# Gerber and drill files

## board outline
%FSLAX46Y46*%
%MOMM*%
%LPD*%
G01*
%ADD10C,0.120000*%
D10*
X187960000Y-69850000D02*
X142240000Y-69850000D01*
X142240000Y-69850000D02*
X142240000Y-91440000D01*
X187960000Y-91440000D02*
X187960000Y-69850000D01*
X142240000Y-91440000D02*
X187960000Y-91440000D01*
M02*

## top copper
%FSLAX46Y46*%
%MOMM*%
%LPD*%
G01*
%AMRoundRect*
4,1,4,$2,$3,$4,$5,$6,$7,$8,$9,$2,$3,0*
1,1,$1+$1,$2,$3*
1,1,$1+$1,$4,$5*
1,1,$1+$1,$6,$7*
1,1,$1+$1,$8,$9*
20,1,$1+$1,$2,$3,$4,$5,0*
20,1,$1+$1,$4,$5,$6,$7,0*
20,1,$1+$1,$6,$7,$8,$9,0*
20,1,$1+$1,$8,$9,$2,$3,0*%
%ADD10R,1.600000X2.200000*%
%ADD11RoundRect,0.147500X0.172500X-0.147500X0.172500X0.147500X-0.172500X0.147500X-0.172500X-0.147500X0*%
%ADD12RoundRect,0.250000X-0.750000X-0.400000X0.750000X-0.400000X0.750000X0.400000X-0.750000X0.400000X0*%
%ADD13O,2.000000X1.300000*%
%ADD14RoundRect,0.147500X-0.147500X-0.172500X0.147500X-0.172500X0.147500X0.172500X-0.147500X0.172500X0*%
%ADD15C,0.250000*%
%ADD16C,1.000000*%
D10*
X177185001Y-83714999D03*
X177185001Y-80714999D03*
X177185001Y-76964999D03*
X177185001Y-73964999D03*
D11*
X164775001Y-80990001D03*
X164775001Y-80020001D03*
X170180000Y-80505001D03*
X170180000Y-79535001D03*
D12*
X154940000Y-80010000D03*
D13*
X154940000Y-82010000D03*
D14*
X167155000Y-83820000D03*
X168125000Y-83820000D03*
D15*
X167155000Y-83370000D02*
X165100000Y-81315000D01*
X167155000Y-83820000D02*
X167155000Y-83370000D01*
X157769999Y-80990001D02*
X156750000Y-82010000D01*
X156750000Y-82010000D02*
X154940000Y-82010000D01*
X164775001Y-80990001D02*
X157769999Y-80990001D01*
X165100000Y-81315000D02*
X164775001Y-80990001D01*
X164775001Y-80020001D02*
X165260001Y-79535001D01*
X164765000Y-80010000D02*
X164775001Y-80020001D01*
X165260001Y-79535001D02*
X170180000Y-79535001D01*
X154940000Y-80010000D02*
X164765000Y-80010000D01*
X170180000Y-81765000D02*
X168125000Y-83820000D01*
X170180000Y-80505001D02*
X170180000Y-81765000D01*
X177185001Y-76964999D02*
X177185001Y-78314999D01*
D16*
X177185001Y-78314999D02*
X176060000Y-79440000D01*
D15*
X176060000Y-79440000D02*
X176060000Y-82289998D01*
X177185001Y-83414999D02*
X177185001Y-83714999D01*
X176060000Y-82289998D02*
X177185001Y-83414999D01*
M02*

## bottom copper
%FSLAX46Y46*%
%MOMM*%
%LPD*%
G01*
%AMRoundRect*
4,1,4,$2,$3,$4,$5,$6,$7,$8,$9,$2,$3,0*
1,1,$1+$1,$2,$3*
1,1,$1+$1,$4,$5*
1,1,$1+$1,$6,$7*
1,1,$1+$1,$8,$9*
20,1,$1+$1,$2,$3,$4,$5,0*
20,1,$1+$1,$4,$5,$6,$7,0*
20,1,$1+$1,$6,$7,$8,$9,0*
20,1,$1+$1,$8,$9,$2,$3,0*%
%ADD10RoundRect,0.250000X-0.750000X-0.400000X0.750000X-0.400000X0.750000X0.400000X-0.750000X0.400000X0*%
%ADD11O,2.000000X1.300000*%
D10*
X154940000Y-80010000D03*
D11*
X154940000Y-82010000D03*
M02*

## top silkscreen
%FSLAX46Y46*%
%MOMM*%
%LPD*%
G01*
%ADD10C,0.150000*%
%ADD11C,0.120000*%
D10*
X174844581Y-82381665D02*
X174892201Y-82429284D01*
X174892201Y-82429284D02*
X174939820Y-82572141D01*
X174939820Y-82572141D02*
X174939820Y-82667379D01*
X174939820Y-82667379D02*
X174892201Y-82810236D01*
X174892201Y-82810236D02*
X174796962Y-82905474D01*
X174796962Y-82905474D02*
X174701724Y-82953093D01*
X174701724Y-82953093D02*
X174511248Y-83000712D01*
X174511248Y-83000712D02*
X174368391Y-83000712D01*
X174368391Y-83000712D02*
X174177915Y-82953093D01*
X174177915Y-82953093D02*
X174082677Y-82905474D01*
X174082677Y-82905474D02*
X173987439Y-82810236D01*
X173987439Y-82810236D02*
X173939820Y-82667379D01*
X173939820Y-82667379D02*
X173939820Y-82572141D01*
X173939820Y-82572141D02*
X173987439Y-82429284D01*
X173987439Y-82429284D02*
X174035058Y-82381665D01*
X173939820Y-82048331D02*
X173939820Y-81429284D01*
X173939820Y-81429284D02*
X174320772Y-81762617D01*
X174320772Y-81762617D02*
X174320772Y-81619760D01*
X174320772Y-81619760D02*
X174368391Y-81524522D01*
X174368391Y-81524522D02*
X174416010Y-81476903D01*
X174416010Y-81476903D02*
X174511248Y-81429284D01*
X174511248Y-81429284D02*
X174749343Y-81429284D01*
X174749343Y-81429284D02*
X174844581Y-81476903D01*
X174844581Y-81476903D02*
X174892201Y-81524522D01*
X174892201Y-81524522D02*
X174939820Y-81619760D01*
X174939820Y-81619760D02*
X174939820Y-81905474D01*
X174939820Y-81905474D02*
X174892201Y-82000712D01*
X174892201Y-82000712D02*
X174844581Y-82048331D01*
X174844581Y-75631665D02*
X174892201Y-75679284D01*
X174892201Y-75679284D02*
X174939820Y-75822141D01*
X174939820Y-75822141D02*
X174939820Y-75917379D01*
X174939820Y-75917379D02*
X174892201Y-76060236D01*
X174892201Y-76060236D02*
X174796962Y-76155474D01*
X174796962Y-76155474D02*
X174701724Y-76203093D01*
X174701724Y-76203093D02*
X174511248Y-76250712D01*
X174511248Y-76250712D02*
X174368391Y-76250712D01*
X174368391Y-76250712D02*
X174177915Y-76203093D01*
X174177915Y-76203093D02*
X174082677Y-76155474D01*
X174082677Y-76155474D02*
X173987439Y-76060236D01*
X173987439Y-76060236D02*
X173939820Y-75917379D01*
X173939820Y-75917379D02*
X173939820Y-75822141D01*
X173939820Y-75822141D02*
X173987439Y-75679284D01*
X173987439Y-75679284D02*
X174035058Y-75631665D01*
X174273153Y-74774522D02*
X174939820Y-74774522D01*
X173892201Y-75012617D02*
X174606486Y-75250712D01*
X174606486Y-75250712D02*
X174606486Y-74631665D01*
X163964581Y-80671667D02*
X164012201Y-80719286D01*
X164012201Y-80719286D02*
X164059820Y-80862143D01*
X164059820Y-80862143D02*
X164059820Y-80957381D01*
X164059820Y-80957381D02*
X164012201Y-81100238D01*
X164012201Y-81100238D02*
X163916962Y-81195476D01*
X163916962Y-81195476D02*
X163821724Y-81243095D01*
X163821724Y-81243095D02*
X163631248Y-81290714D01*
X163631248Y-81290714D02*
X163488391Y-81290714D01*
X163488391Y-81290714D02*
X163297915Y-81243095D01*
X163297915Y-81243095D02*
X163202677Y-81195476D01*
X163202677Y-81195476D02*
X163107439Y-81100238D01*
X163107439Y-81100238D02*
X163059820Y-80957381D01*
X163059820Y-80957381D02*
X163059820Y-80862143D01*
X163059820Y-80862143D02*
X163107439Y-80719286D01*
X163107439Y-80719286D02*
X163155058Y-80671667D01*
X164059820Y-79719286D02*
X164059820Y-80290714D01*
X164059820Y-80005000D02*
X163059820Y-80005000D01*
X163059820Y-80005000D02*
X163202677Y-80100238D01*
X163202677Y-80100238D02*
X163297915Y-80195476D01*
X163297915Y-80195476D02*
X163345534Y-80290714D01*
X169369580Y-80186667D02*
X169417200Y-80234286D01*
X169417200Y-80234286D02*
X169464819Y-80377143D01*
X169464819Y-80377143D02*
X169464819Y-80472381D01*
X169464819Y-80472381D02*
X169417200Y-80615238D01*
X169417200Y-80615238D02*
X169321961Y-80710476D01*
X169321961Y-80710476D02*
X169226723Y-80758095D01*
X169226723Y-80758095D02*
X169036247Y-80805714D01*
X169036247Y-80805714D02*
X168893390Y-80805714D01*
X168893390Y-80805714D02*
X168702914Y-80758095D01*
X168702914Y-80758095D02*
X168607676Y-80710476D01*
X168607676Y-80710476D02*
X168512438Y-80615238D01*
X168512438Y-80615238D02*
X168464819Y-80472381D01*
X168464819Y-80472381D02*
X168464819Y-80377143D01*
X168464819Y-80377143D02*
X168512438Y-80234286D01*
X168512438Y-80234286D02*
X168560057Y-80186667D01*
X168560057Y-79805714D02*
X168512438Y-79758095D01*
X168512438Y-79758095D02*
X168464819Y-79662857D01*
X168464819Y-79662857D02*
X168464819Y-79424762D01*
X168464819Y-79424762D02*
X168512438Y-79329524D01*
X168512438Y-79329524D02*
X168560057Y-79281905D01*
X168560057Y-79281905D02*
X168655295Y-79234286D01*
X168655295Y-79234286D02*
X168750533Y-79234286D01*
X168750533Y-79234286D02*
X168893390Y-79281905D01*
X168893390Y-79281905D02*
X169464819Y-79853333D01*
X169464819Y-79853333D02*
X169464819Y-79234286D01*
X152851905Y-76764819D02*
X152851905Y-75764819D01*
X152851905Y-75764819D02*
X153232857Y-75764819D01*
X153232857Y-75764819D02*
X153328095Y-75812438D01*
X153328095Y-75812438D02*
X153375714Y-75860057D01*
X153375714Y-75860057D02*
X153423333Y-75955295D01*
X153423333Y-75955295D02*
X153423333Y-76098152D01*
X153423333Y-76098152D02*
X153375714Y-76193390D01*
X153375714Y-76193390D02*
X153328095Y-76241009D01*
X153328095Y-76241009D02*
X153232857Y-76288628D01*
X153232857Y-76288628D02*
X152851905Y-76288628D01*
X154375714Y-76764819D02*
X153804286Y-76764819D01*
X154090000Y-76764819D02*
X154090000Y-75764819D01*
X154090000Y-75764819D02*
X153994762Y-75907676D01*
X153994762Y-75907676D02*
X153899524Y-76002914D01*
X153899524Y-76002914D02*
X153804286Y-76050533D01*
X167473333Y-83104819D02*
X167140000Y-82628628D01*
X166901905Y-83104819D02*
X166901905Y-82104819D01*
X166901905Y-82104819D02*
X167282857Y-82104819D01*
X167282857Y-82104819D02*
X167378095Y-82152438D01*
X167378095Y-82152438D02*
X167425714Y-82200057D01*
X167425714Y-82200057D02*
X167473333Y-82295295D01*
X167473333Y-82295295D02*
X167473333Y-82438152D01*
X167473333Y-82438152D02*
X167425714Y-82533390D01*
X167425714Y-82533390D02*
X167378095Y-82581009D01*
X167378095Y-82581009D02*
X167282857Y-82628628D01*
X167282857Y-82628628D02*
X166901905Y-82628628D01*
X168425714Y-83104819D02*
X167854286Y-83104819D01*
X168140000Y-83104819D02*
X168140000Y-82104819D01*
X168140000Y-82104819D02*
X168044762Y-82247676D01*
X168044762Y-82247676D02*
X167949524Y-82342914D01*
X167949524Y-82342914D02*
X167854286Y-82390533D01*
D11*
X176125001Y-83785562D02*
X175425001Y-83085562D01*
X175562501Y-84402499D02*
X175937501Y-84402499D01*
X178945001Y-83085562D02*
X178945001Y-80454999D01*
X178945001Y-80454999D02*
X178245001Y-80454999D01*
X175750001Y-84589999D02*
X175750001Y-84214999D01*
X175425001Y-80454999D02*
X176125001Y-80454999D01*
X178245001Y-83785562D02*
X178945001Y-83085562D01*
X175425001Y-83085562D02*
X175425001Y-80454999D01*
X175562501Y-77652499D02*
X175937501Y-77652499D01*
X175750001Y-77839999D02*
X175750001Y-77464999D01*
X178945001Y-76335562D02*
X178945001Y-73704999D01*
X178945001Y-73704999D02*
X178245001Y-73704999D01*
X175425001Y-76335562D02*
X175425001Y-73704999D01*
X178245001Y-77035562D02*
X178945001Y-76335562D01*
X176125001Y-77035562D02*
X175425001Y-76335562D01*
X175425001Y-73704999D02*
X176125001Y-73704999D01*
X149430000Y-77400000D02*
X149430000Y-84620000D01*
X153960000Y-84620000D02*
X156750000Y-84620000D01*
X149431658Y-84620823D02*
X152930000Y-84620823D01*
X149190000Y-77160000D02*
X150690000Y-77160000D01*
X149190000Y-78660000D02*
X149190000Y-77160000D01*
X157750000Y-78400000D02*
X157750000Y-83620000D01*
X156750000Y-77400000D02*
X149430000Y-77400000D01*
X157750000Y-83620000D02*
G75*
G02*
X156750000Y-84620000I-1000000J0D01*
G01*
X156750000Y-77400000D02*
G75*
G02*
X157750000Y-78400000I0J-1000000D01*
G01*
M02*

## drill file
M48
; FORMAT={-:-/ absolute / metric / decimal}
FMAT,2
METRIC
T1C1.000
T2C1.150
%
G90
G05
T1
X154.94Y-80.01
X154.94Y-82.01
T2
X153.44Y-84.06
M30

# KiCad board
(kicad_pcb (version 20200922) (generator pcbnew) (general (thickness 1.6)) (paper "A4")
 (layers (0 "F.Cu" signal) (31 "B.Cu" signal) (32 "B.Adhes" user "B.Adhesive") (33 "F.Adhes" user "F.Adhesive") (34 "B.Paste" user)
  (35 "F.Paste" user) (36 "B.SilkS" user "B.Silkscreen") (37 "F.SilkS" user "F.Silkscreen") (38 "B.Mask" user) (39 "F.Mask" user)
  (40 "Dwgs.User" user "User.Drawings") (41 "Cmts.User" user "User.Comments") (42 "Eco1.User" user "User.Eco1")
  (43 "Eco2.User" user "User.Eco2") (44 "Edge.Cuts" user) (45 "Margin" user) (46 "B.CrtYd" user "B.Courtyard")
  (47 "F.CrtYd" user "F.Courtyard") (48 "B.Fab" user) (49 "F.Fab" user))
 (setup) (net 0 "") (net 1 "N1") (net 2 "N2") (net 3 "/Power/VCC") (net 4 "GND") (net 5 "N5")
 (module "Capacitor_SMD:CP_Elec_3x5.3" (layer "F.Cu") (at 177.185001 82.214999 90)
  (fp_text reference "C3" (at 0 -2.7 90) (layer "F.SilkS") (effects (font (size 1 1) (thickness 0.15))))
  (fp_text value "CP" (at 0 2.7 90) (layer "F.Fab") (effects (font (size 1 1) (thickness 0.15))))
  (fp_line (start -1.570563 -1.06) (end -0.870563 -1.76) (layer "F.SilkS") (width 0.12))
  (fp_line (start -2.1875 -1.6225) (end -2.1875 -1.2475) (layer "F.SilkS") (width 0.12))
  (fp_line (start -0.870563 1.76) (end 1.76 1.76) (layer "F.SilkS") (width 0.12))
  (fp_line (start 1.76 1.76) (end 1.76 1.06) (layer "F.SilkS") (width 0.12))
  (fp_line (start -2.375 -1.435) (end -2 -1.435) (layer "F.SilkS") (width 0.12))
  (fp_line (start 1.76 -1.76) (end 1.76 -1.06) (layer "F.SilkS") (width 0.12))
  (fp_line (start -1.570563 1.06) (end -0.870563 1.76) (layer "F.SilkS") (width 0.12))
  (fp_line (start -0.870563 -1.76) (end 1.76 -1.76) (layer "F.SilkS") (width 0.12))
  (pad "1" smd rect (at -1.5 0 90) (size 2.2 1.6) (layers "F.Cu" "F.Paste" "F.Mask") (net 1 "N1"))
  (pad "2" smd rect (at 1.5 0 90) (size 2.2 1.6) (layers "F.Cu" "F.Paste" "F.Mask") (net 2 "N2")))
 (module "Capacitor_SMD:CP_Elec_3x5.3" (layer "F.Cu") (at 177.185001 75.464999 90)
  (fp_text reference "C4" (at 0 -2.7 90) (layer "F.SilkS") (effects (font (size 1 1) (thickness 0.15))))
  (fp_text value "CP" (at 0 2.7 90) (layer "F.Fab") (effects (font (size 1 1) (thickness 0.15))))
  (fp_line (start -2.1875 -1.6225) (end -2.1875 -1.2475) (layer "F.SilkS") (width 0.12))
  (fp_line (start -2.375 -1.435) (end -2 -1.435) (layer "F.SilkS") (width 0.12))
  (fp_line (start -0.870563 1.76) (end 1.76 1.76) (layer "F.SilkS") (width 0.12))
  (fp_line (start 1.76 1.76) (end 1.76 1.06) (layer "F.SilkS") (width 0.12))
  (fp_line (start -0.870563 -1.76) (end 1.76 -1.76) (layer "F.SilkS") (width 0.12))
  (fp_line (start -1.570563 1.06) (end -0.870563 1.76) (layer "F.SilkS") (width 0.12))
  (fp_line (start -1.570563 -1.06) (end -0.870563 -1.76) (layer "F.SilkS") (width 0.12))
  (fp_line (start 1.76 -1.76) (end 1.76 -1.06) (layer "F.SilkS") (width 0.12))
  (pad "1" smd rect (at -1.5 0 90) (size 2.2 1.6) (layers "F.Cu" "F.Paste" "F.Mask") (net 1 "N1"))
  (pad "2" smd rect (at 1.5 0 90) (size 2.2 1.6) (layers "F.Cu" "F.Paste" "F.Mask") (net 2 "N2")))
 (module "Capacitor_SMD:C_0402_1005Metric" (layer "F.Cu") (at 164.775001 80.505001 90)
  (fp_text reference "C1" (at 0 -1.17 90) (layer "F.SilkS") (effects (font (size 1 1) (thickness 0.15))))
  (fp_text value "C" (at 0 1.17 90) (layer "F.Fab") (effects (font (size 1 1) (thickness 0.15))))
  (pad "1" smd roundrect (at -0.485 0 90) (size 0.59 0.64) (layers "F.Cu" "F.Paste" "F.Mask") (roundrect_rratio 0.25) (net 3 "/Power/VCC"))
  (pad "2" smd roundrect (at 0.485 0 90) (size 0.59 0.64) (layers "F.Cu" "F.Paste" "F.Mask") (roundrect_rratio 0.25) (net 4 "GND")))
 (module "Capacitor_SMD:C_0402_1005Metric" (layer "F.Cu") (at 170.18 80.020001 90)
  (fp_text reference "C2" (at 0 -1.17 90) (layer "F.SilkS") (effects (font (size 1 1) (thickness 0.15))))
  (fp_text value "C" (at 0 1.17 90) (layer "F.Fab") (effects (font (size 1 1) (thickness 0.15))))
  (pad "1" smd roundrect (at -0.485 0 90) (size 0.59 0.64) (layers "F.Cu" "F.Paste" "F.Mask") (roundrect_rratio 0.25) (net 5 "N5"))
  (pad "2" smd roundrect (at 0.485 0 90) (size 0.59 0.64) (layers "F.Cu" "F.Paste" "F.Mask") (roundrect_rratio 0.25) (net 4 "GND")))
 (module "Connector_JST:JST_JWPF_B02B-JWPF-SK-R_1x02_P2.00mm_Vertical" (layer "F.Cu") (at 154.94 80.01)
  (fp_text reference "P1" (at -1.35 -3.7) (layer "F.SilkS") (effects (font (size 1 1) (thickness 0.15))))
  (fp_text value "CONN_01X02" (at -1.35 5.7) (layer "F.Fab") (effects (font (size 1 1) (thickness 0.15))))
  (fp_line (start -5.51 -2.61) (end -5.51 4.61) (layer "F.SilkS") (width 0.12))
  (fp_line (start -0.98 4.61) (end 1.81 4.61) (layer "F.SilkS") (width 0.12))
  (fp_line (start -5.508342 4.610823) (end -2.01 4.610823) (layer "F.SilkS") (width 0.12))
  (fp_line (start -5.75 -2.85) (end -4.25 -2.85) (layer "F.SilkS") (width 0.12))
  (fp_line (start -5.75 -1.35) (end -5.75 -2.85) (layer "F.SilkS") (width 0.12))
  (fp_line (start 2.81 -1.61) (end 2.81 3.61) (layer "F.SilkS") (width 0.12))
  (fp_line (start 1.81 -2.61) (end -5.51 -2.61) (layer "F.SilkS") (width 0.12))
  (fp_arc (start 1.81 3.61) (end 2.81 3.61) (angle 90) (layer "F.SilkS") (width 0.12))
  (fp_arc (start 1.81 -1.61) (end 1.81 -2.61) (angle 90) (layer "F.SilkS") (width 0.12))
  (pad "" np_thru_hole circle (at -1.5 4.05) (size 1.15 1.15) (drill 1.15) (layers *.Cu *.Mask))
  (pad "1" thru_hole roundrect (at 0 0) (size 2 1.3) (drill 1) (layers *.Cu *.Mask) (roundrect_rratio 0.192308) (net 4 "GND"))
  (pad "2" thru_hole oval (at 0 2) (size 2 1.3) (drill 1) (layers *.Cu *.Mask) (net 3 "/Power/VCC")))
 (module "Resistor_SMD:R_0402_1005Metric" (layer "F.Cu") (at 167.64 83.82)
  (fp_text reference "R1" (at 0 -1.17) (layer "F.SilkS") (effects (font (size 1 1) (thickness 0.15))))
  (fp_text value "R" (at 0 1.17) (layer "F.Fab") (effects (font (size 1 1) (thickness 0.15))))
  (pad "1" smd roundrect (at -0.485 0) (size 0.59 0.64) (layers "F.Cu" "F.Paste" "F.Mask") (roundrect_rratio 0.25) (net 3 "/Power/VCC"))
  (pad "2" smd roundrect (at 0.485 0) (size 0.59 0.64) (layers "F.Cu" "F.Paste" "F.Mask") (roundrect_rratio 0.25) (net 5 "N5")))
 (gr_line (start 187.96 69.85) (end 142.24 69.85) (layer "Edge.Cuts") (width 0.12))
 (gr_line (start 142.24 69.85) (end 142.24 91.44) (layer "Edge.Cuts") (width 0.12))
 (gr_line (start 187.96 91.44) (end 187.96 69.85) (layer "Edge.Cuts") (width 0.12))
 (gr_line (start 142.24 91.44) (end 187.96 91.44) (layer "Edge.Cuts") (width 0.12))
 (segment (start 167.155 83.37) (end 165.1 81.315) (width 0.25) (layer "F.Cu") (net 3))
 (segment (start 167.155 83.82) (end 167.155 83.37) (width 0.25) (layer "F.Cu") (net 3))
 (segment (start 157.769999 80.990001) (end 156.75 82.01) (width 0.25) (layer "F.Cu") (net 3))
 (segment (start 156.75 82.01) (end 154.94 82.01) (width 0.25) (layer "F.Cu") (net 3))
 (segment (start 164.775001 80.990001) (end 157.769999 80.990001) (width 0.25) (layer "F.Cu") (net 3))
 (segment (start 165.1 81.315) (end 164.775001 80.990001) (width 0.25) (layer "F.Cu") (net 3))
 (segment (start 164.775001 80.020001) (end 165.260001 79.535001) (width 0.25) (layer "F.Cu") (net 4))
 (segment (start 164.765 80.01) (end 164.775001 80.020001) (width 0.25) (layer "F.Cu") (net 4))
 (segment (start 165.260001 79.535001) (end 170.18 79.535001) (width 0.25) (layer "F.Cu") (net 4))
 (segment (start 154.94 80.01) (end 164.765 80.01) (width 0.25) (layer "F.Cu") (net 4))
 (segment (start 170.18 81.765) (end 168.125 83.82) (width 0.25) (layer "F.Cu") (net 5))
 (segment (start 170.18 80.505001) (end 170.18 81.765) (width 0.25) (layer "F.Cu") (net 5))
 (segment (start 177.185001 76.964999) (end 177.185001 78.314999) (width 0.25) (layer "F.Cu") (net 1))
 (segment (start 177.185001 78.314999) (end 176.06 79.44) (width 1) (layer "F.Cu") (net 1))
 (segment (start 176.06 79.44) (end 176.06 82.289998) (width 0.25) (layer "F.Cu") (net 1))
 (segment (start 177.185001 83.414999) (end 177.185001 83.714999) (width 0.25) (layer "F.Cu") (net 1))
 (segment (start 176.06 82.289998) (end 177.185001 83.414999) (width 0.25) (layer "F.Cu") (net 1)))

